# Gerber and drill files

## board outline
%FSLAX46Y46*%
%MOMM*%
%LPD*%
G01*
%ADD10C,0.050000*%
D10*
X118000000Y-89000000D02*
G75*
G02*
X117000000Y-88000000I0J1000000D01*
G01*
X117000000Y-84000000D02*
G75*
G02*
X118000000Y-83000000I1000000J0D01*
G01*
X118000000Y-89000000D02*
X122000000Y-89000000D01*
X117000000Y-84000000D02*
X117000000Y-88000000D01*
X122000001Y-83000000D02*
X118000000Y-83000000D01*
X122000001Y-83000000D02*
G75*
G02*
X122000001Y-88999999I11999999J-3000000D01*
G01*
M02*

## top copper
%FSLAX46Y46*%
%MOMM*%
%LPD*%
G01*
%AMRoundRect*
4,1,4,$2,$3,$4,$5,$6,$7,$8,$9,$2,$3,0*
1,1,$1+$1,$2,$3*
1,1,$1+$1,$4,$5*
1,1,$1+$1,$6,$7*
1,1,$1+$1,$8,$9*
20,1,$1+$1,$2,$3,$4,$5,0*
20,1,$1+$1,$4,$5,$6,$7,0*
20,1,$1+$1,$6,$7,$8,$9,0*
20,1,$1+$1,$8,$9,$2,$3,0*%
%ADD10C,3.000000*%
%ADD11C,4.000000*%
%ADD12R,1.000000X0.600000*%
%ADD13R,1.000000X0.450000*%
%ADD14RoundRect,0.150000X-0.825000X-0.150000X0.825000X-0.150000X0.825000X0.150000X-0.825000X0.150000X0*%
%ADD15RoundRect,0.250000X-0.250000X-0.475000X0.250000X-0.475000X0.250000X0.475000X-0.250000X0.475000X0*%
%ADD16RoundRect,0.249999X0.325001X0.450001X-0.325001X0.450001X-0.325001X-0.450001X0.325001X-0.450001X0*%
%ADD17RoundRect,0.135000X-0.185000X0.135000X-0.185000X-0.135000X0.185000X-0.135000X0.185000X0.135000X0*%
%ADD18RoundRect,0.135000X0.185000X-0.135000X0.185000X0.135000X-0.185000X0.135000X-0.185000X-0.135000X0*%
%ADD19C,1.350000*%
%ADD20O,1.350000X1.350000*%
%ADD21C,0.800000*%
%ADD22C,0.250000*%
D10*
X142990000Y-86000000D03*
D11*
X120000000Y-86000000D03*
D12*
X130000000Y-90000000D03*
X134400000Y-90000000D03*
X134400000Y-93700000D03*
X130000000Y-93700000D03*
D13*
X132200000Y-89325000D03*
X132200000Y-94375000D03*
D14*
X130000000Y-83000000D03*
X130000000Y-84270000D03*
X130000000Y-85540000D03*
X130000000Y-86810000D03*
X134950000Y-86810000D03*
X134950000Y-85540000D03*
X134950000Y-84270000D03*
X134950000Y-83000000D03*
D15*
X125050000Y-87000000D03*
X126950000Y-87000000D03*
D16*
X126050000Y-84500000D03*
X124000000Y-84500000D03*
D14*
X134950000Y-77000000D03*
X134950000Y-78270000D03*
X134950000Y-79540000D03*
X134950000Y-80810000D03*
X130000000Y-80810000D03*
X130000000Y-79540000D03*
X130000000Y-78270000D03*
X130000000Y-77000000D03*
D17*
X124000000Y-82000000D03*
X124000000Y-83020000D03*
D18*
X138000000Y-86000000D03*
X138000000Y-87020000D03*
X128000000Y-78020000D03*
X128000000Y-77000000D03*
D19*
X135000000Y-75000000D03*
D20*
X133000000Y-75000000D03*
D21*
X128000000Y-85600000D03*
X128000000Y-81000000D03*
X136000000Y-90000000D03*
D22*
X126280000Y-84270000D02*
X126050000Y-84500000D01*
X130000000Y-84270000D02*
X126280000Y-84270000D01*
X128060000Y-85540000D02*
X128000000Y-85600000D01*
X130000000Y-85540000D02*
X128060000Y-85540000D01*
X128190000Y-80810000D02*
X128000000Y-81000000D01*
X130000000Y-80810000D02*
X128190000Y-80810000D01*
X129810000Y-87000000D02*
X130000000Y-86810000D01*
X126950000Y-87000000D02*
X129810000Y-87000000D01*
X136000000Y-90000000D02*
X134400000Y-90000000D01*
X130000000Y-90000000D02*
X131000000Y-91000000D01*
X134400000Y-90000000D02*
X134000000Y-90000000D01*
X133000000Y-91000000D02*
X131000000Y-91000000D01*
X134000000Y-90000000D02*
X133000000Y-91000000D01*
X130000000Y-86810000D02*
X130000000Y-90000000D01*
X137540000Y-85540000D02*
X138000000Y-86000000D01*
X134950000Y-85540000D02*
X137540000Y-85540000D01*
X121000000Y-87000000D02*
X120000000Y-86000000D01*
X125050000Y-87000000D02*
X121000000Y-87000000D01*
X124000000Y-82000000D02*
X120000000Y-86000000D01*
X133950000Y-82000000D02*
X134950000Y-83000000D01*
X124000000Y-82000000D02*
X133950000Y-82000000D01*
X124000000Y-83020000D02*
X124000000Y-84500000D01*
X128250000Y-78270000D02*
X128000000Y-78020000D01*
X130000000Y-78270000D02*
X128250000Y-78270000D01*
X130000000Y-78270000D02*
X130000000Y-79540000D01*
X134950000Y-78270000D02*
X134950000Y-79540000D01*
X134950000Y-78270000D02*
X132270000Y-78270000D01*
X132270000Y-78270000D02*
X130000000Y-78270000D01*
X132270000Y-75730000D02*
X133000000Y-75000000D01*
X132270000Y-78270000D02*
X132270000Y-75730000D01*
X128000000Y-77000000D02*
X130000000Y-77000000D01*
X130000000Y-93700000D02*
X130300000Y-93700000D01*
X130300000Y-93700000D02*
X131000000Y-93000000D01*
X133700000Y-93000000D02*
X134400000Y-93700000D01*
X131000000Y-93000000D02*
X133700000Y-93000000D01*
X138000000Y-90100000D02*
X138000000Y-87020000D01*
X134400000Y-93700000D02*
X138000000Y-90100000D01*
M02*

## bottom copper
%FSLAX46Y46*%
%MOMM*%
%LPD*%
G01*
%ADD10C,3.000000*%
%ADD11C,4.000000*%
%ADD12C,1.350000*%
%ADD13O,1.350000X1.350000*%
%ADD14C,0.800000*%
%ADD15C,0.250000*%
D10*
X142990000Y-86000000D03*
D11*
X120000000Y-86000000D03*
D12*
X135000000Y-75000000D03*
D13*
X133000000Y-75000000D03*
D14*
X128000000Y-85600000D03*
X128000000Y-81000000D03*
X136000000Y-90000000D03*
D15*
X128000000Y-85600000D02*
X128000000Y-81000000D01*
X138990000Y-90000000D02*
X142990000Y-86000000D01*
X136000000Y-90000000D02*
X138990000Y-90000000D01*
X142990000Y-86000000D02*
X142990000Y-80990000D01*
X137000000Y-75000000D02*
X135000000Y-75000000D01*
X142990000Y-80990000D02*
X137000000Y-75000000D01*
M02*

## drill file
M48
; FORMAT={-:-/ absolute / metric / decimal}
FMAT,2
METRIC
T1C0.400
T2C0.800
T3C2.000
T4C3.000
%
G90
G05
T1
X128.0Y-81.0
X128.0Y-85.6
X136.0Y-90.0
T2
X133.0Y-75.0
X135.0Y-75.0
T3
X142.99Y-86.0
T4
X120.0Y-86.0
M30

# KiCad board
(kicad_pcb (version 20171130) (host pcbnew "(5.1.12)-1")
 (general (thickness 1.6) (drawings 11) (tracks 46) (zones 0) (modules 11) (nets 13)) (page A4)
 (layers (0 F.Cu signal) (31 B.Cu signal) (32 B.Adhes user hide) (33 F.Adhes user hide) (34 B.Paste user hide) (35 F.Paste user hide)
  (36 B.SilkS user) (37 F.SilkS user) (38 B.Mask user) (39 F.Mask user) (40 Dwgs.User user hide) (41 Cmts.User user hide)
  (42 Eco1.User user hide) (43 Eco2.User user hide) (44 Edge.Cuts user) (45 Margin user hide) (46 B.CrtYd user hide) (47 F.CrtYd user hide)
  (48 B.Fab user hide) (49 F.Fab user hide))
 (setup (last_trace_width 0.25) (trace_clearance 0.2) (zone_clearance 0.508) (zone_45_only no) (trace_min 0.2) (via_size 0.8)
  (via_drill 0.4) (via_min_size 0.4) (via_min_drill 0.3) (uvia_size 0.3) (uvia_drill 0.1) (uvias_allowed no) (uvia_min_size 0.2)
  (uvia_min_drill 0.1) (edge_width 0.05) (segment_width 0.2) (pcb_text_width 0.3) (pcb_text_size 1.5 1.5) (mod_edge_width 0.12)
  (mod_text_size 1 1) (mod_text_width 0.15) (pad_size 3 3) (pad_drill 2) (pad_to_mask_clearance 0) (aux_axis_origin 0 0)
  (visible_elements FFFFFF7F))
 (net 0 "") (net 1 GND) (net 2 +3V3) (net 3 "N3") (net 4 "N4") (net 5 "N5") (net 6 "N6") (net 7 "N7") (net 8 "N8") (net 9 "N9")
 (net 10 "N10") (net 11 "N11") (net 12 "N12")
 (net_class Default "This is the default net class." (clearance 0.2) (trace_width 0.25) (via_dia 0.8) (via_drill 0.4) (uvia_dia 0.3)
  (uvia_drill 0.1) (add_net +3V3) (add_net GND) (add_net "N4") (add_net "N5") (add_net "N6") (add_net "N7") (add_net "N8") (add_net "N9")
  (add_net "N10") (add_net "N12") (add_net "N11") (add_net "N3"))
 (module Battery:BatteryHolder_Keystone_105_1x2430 (layer F.Cu) (at 120 86)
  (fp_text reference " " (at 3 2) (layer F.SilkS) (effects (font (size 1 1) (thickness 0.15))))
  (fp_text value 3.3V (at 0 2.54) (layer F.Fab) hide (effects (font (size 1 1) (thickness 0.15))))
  (pad 2 thru_hole circle (at 22.99 0) (size 3 3) (drill 2) (layers *.Cu *.Mask) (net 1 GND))
  (pad 1 thru_hole circle (at 0 0) (size 4 4) (drill 3) (layers *.Cu *.Mask) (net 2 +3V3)))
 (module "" (layer F.Cu) (at 146 87)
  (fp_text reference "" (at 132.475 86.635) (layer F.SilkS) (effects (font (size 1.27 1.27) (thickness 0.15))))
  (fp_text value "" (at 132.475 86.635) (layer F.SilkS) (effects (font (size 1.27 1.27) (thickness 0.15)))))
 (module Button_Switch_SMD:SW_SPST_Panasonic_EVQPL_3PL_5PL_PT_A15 (layer F.Cu) (at 132.2 91.85 270)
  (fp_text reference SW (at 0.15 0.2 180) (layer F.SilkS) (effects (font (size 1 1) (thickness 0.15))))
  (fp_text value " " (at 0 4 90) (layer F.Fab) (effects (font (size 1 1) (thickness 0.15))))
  (pad 1 smd rect (at -1.85 2.2 270) (size 0.6 1) (layers F.Cu F.Paste F.Mask) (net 1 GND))
  (pad 1 smd rect (at -1.85 -2.2 270) (size 0.6 1) (layers F.Cu F.Paste F.Mask) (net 1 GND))
  (pad 2 smd rect (at 1.85 -2.2 270) (size 0.6 1) (layers F.Cu F.Paste F.Mask) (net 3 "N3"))
  (pad 2 smd rect (at 1.85 2.2 270) (size 0.6 1) (layers F.Cu F.Paste F.Mask) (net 3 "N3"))
  (pad 0 smd rect (at -2.525 0 270) (size 0.45 1) (layers F.Cu F.Paste F.Mask))
  (pad 0 smd rect (at 2.525 0 270) (size 0.45 1) (layers F.Cu F.Paste F.Mask)))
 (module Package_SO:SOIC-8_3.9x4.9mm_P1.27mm (layer F.Cu) (at 132.475 84.905)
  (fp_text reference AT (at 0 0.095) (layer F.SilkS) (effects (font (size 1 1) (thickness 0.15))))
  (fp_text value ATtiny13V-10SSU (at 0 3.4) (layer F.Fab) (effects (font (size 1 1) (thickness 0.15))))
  (pad 1 smd roundrect (at -2.475 -1.905) (size 1.95 0.6) (layers F.Cu F.Paste F.Mask) (roundrect_rratio 0.25) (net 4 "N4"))
  (pad 2 smd roundrect (at -2.475 -0.635) (size 1.95 0.6) (layers F.Cu F.Paste F.Mask) (roundrect_rratio 0.25) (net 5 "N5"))
  (pad 3 smd roundrect (at -2.475 0.635) (size 1.95 0.6) (layers F.Cu F.Paste F.Mask) (roundrect_rratio 0.25) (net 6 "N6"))
  (pad 4 smd roundrect (at -2.475 1.905) (size 1.95 0.6) (layers F.Cu F.Paste F.Mask) (roundrect_rratio 0.25) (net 1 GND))
  (pad 5 smd roundrect (at 2.475 1.905) (size 1.95 0.6) (layers F.Cu F.Paste F.Mask) (roundrect_rratio 0.25) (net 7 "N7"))
  (pad 6 smd roundrect (at 2.475 0.635) (size 1.95 0.6) (layers F.Cu F.Paste F.Mask) (roundrect_rratio 0.25) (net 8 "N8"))
  (pad 7 smd roundrect (at 2.475 -0.635) (size 1.95 0.6) (layers F.Cu F.Paste F.Mask) (roundrect_rratio 0.25) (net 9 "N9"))
  (pad 8 smd roundrect (at 2.475 -1.905) (size 1.95 0.6) (layers F.Cu F.Paste F.Mask) (roundrect_rratio 0.25) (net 2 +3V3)))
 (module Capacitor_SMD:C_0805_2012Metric (layer F.Cu) (at 126 87)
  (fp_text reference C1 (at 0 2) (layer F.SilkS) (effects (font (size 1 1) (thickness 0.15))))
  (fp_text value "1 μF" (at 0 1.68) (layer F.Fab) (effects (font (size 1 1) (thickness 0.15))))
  (pad 1 smd roundrect (at -0.95 0) (size 1 1.45) (layers F.Cu F.Paste F.Mask) (roundrect_rratio 0.25) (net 2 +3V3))
  (pad 2 smd roundrect (at 0.95 0) (size 1 1.45) (layers F.Cu F.Paste F.Mask) (roundrect_rratio 0.25) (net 1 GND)))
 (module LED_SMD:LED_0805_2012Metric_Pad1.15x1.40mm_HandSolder (layer F.Cu) (at 125.025 84.5 180)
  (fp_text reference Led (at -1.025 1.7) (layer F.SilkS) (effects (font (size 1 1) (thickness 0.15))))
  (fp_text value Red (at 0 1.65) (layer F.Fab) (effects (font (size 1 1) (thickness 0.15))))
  (pad 1 smd roundrect (at -1.025 0 180) (size 1.15 1.4) (layers F.Cu F.Paste F.Mask) (roundrect_rratio 0.2173904347826087) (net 5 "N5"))
  (pad 2 smd roundrect (at 1.025 0 180) (size 1.15 1.4) (layers F.Cu F.Paste F.Mask) (roundrect_rratio 0.2173904347826087) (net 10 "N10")))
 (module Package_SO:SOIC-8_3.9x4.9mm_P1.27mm (layer F.Cu) (at 132.475 78.905)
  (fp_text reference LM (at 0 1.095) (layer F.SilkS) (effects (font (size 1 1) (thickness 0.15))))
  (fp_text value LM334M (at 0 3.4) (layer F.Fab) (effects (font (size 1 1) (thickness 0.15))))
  (pad 8 smd roundrect (at 2.475 -1.905) (size 1.95 0.6) (layers F.Cu F.Paste F.Mask) (roundrect_rratio 0.25))
  (pad 7 smd roundrect (at 2.475 -0.635) (size 1.95 0.6) (layers F.Cu F.Paste F.Mask) (roundrect_rratio 0.25) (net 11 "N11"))
  (pad 6 smd roundrect (at 2.475 0.635) (size 1.95 0.6) (layers F.Cu F.Paste F.Mask) (roundrect_rratio 0.25) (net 11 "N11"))
  (pad 5 smd roundrect (at 2.475 1.905) (size 1.95 0.6) (layers F.Cu F.Paste F.Mask) (roundrect_rratio 0.25))
  (pad 4 smd roundrect (at -2.475 1.905) (size 1.95 0.6) (layers F.Cu F.Paste F.Mask) (roundrect_rratio 0.25) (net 6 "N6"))
  (pad 3 smd roundrect (at -2.475 0.635) (size 1.95 0.6) (layers F.Cu F.Paste F.Mask) (roundrect_rratio 0.25) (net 11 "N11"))
  (pad 2 smd roundrect (at -2.475 -0.635) (size 1.95 0.6) (layers F.Cu F.Paste F.Mask) (roundrect_rratio 0.25) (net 11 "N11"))
  (pad 1 smd roundrect (at -2.475 -1.905) (size 1.95 0.6) (layers F.Cu F.Paste F.Mask) (roundrect_rratio 0.25) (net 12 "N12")))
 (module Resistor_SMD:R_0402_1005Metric (layer F.Cu) (at 124 82.51 270)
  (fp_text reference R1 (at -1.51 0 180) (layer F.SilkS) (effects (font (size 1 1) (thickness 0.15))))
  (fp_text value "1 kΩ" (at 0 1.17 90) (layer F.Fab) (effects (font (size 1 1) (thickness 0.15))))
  (pad 1 smd roundrect (at -0.51 0 270) (size 0.54 0.64) (layers F.Cu F.Paste F.Mask) (roundrect_rratio 0.25) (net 2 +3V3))
  (pad 2 smd roundrect (at 0.51 0 270) (size 0.54 0.64) (layers F.Cu F.Paste F.Mask) (roundrect_rratio 0.25) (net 10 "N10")))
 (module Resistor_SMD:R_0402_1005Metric (layer F.Cu) (at 138 86.51 90)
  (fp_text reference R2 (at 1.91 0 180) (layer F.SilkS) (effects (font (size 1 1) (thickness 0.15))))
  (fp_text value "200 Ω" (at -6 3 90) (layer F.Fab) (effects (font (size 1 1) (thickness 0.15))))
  (pad 2 smd roundrect (at 0.51 0 90) (size 0.54 0.64) (layers F.Cu F.Paste F.Mask) (roundrect_rratio 0.25) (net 8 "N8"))
  (pad 1 smd roundrect (at -0.51 0 90) (size 0.54 0.64) (layers F.Cu F.Paste F.Mask) (roundrect_rratio 0.25) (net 3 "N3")))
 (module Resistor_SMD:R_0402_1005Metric (layer F.Cu) (at 128 77.51 90)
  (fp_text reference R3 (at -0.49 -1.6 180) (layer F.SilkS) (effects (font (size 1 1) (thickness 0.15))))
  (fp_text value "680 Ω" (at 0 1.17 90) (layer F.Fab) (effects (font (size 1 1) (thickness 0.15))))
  (pad 1 smd roundrect (at -0.51 0 90) (size 0.54 0.64) (layers F.Cu F.Paste F.Mask) (roundrect_rratio 0.25) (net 11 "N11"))
  (pad 2 smd roundrect (at 0.51 0 90) (size 0.54 0.64) (layers F.Cu F.Paste F.Mask) (roundrect_rratio 0.25) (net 12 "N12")))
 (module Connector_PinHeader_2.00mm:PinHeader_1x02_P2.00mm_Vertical (layer F.Cu) (at 135 75 270)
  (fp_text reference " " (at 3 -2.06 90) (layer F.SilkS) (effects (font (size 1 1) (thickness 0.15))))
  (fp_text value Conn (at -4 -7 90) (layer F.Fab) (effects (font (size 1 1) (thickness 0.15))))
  (pad 1 thru_hole circle (at 0 0 270) (size 1.35 1.35) (drill 0.8) (layers *.Cu *.Mask) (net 1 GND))
  (pad 2 thru_hole oval (at 0 2 270) (size 1.35 1.35) (drill 0.8) (layers *.Cu *.Mask) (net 11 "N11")))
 (gr_arc (start 118 88) (end 117 88) (angle -90) (layer Edge.Cuts) (width 0.05))
 (gr_arc (start 118 84) (end 118 83) (angle -90) (layer Edge.Cuts) (width 0.05))
 (gr_line (start 118 89) (end 122 89) (layer Edge.Cuts) (width 0.05))
 (gr_line (start 117 84) (end 117 88) (layer Edge.Cuts) (width 0.05))
 (gr_line (start 122.000001 83) (end 118 83) (layer Edge.Cuts) (width 0.05))
 (gr_arc (start 134 86) (end 122.000001 88.999999) (angle -331.9275131) (layer Edge.Cuts) (width 0.05))
 (segment (start 126.28 84.27) (end 126.05 84.5) (width 0.25) (layer F.Cu) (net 5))
 (segment (start 130 84.27) (end 126.28 84.27) (width 0.25) (layer F.Cu) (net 5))
 (via (at 128 85.6) (size 0.8) (drill 0.4) (layers F.Cu B.Cu) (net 6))
 (segment (start 128.06 85.54) (end 128 85.6) (width 0.25) (layer F.Cu) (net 6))
 (segment (start 130 85.54) (end 128.06 85.54) (width 0.25) (layer F.Cu) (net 6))
 (via (at 128 81) (size 0.8) (drill 0.4) (layers F.Cu B.Cu) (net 6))
 (segment (start 128 85.6) (end 128 81) (width 0.25) (layer B.Cu) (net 6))
 (segment (start 128.19 80.81) (end 128 81) (width 0.25) (layer F.Cu) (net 6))
 (segment (start 130 80.81) (end 128.19 80.81) (width 0.25) (layer F.Cu) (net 6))
 (segment (start 129.81 87) (end 130 86.81) (width 0.25) (layer F.Cu) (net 1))
 (segment (start 126.95 87) (end 129.81 87) (width 0.25) (layer F.Cu) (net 1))
 (segment (start 136 90) (end 134.4 90) (width 0.25) (layer F.Cu) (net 1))
 (via (at 136 90) (size 0.8) (drill 0.4) (layers F.Cu B.Cu) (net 1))
 (segment (start 130 90) (end 131 91) (width 0.25) (layer F.Cu) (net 1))
 (segment (start 134.4 90) (end 134 90) (width 0.25) (layer F.Cu) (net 1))
 (segment (start 133 91) (end 131 91) (width 0.25) (layer F.Cu) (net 1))
 (segment (start 134 90) (end 133 91) (width 0.25) (layer F.Cu) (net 1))
 (segment (start 130 86.81) (end 130 90) (width 0.25) (layer F.Cu) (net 1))
 (segment (start 138.99 90) (end 142.99 86) (width 0.25) (layer B.Cu) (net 1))
 (segment (start 136 90) (end 138.99 90) (width 0.25) (layer B.Cu) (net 1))
 (segment (start 142.99 86) (end 142.99 80.99) (width 0.25) (layer B.Cu) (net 1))
 (segment (start 137 75) (end 135 75) (width 0.25) (layer B.Cu) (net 1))
 (segment (start 142.99 80.99) (end 137 75) (width 0.25) (layer B.Cu) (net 1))
 (segment (start 137.54 85.54) (end 138 86) (width 0.25) (layer F.Cu) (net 8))
 (segment (start 134.95 85.54) (end 137.54 85.54) (width 0.25) (layer F.Cu) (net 8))
 (segment (start 121 87) (end 120 86) (width 0.25) (layer F.Cu) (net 2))
 (segment (start 125.05 87) (end 121 87) (width 0.25) (layer F.Cu) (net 2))
 (segment (start 124 82) (end 120 86) (width 0.25) (layer F.Cu) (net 2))
 (segment (start 133.95 82) (end 134.95 83) (width 0.25) (layer F.Cu) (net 2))
 (segment (start 124 82) (end 133.95 82) (width 0.25) (layer F.Cu) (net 2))
 (segment (start 124 83.02) (end 124 84.5) (width 0.25) (layer F.Cu) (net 10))
 (segment (start 128.25 78.27) (end 128 78.02) (width 0.25) (layer F.Cu) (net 11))
 (segment (start 130 78.27) (end 128.25 78.27) (width 0.25) (layer F.Cu) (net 11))
 (segment (start 130 78.27) (end 130 79.54) (width 0.25) (layer F.Cu) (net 11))
 (segment (start 134.95 78.27) (end 134.95 79.54) (width 0.25) (layer F.Cu) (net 11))
 (segment (start 134.95 78.27) (end 132.27 78.27) (width 0.25) (layer F.Cu) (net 11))
 (segment (start 132.27 78.27) (end 130 78.27) (width 0.25) (layer F.Cu) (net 11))
 (segment (start 132.27 75.73) (end 133 75) (width 0.25) (layer F.Cu) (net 11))
 (segment (start 132.27 78.27) (end 132.27 75.73) (width 0.25) (layer F.Cu) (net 11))
 (segment (start 128 77) (end 130 77) (width 0.25) (layer F.Cu) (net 12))
 (segment (start 130 93.7) (end 130.3 93.7) (width 0.25) (layer F.Cu) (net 3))
 (segment (start 130.3 93.7) (end 131 93) (width 0.25) (layer F.Cu) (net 3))
 (segment (start 133.7 93) (end 134.4 93.7) (width 0.25) (layer F.Cu) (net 3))
 (segment (start 131 93) (end 133.7 93) (width 0.25) (layer F.Cu) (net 3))
 (segment (start 138 90.1) (end 138 87.02) (width 0.25) (layer F.Cu) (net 3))
 (segment (start 134.4 93.7) (end 138 90.1) (width 0.25) (layer F.Cu) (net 3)))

